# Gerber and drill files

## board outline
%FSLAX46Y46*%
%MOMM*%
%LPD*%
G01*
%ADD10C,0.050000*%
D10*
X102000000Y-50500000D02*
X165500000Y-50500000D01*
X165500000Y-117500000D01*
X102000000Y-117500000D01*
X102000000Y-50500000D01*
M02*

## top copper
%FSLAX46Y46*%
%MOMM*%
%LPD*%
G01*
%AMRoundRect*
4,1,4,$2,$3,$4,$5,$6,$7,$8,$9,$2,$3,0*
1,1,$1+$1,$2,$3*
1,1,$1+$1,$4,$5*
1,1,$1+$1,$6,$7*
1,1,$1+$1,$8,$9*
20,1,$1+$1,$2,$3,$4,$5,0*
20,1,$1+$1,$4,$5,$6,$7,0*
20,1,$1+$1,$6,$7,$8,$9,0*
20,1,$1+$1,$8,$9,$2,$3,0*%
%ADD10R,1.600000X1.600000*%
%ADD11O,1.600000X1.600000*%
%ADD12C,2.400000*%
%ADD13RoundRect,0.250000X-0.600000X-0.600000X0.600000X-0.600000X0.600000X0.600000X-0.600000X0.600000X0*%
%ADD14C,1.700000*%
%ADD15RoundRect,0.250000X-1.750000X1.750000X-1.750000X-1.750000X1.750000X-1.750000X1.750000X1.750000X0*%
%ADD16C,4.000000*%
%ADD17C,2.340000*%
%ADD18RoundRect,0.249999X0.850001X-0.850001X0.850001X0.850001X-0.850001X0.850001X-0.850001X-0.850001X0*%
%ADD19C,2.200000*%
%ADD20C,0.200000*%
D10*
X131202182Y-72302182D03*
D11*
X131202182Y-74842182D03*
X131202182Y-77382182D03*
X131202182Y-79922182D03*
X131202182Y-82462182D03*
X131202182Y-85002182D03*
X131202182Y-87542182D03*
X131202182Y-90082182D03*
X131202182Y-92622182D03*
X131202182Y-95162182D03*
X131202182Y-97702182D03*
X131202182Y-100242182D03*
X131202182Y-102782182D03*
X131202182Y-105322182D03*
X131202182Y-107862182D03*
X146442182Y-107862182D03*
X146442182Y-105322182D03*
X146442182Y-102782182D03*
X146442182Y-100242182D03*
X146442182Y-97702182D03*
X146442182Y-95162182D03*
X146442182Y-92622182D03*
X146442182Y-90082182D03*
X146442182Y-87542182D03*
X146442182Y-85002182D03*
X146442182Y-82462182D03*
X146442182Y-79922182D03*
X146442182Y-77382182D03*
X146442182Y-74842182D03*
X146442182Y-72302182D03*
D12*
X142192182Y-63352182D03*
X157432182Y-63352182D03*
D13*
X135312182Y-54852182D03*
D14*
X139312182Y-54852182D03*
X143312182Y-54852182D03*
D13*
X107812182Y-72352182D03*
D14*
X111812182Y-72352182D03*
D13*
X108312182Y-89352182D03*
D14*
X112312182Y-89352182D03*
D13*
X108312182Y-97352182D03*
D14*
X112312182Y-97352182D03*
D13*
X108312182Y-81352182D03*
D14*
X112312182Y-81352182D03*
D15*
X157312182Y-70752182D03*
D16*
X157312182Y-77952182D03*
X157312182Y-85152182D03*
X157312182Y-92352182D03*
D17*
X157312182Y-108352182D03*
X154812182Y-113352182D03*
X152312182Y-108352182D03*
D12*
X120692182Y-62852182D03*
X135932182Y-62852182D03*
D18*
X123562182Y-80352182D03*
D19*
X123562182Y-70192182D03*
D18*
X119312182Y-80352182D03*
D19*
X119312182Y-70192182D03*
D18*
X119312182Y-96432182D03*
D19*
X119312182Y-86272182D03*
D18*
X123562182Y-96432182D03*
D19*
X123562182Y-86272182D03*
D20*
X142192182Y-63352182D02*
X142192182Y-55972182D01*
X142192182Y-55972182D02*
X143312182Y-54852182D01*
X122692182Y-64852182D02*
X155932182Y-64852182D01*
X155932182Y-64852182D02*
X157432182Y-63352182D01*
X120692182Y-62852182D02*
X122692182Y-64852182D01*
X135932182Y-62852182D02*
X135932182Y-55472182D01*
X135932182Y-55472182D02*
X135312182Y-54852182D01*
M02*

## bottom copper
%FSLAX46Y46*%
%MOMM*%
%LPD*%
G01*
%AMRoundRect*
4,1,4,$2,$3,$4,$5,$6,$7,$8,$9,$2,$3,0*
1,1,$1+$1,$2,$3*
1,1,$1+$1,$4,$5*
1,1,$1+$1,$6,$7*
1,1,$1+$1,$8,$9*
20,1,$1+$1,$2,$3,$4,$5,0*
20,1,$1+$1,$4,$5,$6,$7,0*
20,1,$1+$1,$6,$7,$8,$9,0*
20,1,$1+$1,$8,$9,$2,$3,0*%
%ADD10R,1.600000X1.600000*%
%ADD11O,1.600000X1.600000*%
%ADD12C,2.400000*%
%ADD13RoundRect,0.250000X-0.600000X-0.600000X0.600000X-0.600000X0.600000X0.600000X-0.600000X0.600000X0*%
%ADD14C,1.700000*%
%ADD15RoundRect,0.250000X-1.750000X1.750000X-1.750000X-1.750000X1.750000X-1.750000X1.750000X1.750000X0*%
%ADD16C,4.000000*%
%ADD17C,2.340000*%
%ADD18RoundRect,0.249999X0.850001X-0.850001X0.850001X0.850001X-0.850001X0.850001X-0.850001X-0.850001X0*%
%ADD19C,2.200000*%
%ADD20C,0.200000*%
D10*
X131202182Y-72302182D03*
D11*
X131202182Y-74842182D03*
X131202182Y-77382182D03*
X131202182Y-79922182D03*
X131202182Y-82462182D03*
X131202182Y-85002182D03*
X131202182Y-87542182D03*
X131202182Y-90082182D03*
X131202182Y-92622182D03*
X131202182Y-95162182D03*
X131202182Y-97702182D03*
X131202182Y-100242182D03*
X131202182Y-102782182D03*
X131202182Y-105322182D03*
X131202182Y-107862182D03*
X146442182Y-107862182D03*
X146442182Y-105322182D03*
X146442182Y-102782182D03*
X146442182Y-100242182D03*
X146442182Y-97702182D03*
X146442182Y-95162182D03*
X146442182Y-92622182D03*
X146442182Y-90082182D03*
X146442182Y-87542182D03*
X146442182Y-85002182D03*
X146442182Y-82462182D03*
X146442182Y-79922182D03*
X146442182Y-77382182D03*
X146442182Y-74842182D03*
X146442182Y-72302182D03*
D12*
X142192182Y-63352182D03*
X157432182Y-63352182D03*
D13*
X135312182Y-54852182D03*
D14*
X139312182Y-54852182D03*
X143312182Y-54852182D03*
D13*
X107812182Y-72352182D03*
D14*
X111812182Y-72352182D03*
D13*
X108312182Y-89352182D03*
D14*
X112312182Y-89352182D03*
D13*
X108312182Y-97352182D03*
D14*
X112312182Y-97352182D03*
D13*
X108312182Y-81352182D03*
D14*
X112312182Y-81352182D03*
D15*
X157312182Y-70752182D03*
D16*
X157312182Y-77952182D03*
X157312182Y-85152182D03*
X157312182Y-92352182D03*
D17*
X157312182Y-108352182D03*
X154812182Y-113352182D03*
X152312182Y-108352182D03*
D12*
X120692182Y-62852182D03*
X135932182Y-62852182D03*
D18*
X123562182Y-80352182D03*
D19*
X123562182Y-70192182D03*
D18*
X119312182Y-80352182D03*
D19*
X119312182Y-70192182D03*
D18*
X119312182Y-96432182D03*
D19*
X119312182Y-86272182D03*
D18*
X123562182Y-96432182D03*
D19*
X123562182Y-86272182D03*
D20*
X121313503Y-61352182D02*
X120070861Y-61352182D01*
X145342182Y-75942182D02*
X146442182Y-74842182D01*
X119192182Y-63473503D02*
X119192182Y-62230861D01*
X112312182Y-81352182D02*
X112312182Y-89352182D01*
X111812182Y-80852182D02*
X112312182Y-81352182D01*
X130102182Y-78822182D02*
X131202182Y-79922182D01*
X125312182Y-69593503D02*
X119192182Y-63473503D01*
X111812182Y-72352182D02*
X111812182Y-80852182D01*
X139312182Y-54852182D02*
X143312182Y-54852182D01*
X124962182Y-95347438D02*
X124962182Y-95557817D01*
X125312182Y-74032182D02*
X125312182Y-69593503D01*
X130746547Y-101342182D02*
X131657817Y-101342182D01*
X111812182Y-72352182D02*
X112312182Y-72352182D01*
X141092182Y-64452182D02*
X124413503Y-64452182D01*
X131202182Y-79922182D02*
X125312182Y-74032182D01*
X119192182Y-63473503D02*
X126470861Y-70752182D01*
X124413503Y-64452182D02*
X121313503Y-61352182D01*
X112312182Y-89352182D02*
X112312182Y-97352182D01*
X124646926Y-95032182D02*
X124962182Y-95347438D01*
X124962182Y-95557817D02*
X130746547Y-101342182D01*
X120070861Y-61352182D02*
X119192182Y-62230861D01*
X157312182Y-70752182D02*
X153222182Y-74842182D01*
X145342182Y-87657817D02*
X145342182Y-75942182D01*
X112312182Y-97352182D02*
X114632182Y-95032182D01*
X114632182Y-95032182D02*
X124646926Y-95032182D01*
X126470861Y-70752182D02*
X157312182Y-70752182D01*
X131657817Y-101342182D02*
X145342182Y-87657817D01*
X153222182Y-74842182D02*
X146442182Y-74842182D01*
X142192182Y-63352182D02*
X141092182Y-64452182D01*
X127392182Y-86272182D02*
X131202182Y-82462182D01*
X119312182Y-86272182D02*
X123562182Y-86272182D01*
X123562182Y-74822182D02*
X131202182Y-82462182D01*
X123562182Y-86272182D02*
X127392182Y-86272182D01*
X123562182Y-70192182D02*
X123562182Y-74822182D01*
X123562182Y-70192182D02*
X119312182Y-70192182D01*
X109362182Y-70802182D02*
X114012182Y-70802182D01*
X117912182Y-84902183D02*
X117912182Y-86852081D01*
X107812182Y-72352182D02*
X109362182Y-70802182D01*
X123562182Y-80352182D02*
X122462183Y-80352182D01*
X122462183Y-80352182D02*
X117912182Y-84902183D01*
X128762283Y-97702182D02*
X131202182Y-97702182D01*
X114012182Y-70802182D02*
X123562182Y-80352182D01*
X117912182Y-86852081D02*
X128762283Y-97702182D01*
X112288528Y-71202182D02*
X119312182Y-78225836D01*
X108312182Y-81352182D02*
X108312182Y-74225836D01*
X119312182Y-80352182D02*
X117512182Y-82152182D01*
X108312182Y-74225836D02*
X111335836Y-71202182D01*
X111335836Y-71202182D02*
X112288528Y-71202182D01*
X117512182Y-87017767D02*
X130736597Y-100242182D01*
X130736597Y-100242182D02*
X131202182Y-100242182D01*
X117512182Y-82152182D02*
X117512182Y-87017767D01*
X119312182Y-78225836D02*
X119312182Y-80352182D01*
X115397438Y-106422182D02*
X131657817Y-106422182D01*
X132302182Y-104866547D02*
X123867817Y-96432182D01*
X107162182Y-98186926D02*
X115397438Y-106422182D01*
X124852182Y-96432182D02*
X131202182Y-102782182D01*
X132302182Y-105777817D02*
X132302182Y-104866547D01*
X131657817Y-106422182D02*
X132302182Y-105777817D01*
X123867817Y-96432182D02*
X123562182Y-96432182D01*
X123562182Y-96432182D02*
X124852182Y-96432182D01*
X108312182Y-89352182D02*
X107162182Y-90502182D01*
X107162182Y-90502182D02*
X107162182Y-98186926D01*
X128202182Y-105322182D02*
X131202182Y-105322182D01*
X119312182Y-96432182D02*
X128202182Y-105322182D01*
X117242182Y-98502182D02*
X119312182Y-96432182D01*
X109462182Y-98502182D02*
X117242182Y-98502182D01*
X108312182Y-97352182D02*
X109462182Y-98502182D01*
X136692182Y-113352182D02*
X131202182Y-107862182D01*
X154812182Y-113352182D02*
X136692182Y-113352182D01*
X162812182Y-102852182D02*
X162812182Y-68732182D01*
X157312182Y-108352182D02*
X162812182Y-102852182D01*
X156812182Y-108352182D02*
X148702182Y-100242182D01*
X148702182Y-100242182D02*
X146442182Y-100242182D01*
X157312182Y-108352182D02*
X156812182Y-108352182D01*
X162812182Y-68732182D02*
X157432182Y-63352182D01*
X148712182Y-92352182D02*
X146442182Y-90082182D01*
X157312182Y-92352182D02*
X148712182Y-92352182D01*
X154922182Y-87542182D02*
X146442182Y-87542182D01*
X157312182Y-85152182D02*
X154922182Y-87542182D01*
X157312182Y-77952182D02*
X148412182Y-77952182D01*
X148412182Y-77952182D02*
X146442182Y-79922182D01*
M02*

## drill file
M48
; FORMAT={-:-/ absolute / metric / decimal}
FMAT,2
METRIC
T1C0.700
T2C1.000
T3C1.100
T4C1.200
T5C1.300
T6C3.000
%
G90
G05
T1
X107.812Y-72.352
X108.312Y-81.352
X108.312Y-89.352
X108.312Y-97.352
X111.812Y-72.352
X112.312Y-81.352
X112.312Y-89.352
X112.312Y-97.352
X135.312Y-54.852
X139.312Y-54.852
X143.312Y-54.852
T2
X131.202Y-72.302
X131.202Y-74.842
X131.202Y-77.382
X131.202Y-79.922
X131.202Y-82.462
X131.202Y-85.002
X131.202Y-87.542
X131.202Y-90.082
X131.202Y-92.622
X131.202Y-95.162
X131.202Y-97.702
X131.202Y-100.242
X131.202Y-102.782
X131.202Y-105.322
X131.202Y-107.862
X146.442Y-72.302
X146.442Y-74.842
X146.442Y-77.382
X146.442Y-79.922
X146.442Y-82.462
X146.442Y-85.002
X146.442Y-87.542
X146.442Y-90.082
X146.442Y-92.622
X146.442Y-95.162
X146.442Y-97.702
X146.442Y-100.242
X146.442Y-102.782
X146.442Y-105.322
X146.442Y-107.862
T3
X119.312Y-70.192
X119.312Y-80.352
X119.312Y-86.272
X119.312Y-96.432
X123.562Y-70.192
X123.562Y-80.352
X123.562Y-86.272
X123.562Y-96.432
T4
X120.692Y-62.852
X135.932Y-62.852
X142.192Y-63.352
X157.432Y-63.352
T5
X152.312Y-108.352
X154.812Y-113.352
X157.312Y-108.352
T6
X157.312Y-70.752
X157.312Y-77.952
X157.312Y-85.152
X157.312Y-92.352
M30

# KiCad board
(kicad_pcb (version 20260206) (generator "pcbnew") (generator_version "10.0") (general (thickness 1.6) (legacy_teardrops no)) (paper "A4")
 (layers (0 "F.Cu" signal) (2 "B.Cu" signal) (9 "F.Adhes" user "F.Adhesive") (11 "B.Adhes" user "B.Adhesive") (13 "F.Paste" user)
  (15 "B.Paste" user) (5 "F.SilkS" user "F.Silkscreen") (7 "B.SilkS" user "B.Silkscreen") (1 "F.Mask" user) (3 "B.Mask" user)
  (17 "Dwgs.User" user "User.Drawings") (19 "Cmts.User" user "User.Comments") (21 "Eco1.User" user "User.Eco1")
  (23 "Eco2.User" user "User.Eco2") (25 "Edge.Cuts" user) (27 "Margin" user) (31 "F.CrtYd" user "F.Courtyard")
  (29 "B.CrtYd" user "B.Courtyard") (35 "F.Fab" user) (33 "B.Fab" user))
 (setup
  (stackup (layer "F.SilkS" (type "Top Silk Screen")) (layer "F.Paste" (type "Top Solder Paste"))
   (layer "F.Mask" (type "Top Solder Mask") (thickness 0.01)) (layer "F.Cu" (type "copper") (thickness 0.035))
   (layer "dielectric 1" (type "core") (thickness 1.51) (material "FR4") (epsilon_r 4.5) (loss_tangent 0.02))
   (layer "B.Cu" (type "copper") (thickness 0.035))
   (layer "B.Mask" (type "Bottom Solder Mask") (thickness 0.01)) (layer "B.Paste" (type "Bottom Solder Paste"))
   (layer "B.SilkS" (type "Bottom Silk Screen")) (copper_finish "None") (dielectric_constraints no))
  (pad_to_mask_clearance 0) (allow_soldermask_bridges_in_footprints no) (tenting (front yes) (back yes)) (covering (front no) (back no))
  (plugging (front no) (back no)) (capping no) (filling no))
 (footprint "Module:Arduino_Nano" (layer "F.Cu") (at 131.202182 72.302182)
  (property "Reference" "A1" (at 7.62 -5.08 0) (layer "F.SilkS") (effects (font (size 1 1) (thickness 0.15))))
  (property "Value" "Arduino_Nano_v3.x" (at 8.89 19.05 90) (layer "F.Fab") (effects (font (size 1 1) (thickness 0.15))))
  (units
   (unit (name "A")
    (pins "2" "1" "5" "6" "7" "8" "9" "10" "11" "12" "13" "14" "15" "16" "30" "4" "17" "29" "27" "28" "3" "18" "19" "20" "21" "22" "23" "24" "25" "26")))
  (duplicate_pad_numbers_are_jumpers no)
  (pad "1" thru_hole rect (at 0 0) (size 1.6 1.6) (drill 1) (layers "*.Cu" "*.Mask") (remove_unused_layers no)
   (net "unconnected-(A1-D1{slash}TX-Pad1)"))
  (pad "2" thru_hole oval (at 0 2.54) (size 1.6 1.6) (drill 1) (layers "*.Cu" "*.Mask") (remove_unused_layers no)
   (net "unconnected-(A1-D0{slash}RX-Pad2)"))
  (pad "3" thru_hole oval (at 0 5.08) (size 1.6 1.6) (drill 1) (layers "*.Cu" "*.Mask") (remove_unused_layers no)
   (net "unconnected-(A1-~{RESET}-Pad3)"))
  (pad "4" thru_hole oval (at 0 7.62) (size 1.6 1.6) (drill 1) (layers "*.Cu" "*.Mask") (remove_unused_layers no) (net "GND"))
  (pad "5" thru_hole oval (at 0 10.16) (size 1.6 1.6) (drill 1) (layers "*.Cu" "*.Mask") (remove_unused_layers no) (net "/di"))
  (pad "6" thru_hole oval (at 0 12.7) (size 1.6 1.6) (drill 1) (layers "*.Cu" "*.Mask") (remove_unused_layers no)
   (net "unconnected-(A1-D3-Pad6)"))
  (pad "7" thru_hole oval (at 0 15.24) (size 1.6 1.6) (drill 1) (layers "*.Cu" "*.Mask") (remove_unused_layers no)
   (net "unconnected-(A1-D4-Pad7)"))
  (pad "8" thru_hole oval (at 0 17.78) (size 1.6 1.6) (drill 1) (layers "*.Cu" "*.Mask") (remove_unused_layers no)
   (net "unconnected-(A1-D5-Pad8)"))
  (pad "9" thru_hole oval (at 0 20.32) (size 1.6 1.6) (drill 1) (layers "*.Cu" "*.Mask") (remove_unused_layers no)
   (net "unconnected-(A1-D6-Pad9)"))
  (pad "10" thru_hole oval (at 0 22.86) (size 1.6 1.6) (drill 1) (layers "*.Cu" "*.Mask") (remove_unused_layers no)
   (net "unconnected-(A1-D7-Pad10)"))
  (pad "11" thru_hole oval (at 0 25.4) (size 1.6 1.6) (drill 1) (layers "*.Cu" "*.Mask") (remove_unused_layers no) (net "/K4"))
  (pad "12" thru_hole oval (at 0 27.94) (size 1.6 1.6) (drill 1) (layers "*.Cu" "*.Mask") (remove_unused_layers no) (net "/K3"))
  (pad "13" thru_hole oval (at 0 30.48) (size 1.6 1.6) (drill 1) (layers "*.Cu" "*.Mask") (remove_unused_layers no) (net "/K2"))
  (pad "14" thru_hole oval (at 0 33.02) (size 1.6 1.6) (drill 1) (layers "*.Cu" "*.Mask") (remove_unused_layers no) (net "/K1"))
  (pad "15" thru_hole oval (at 0 35.56) (size 1.6 1.6) (drill 1) (layers "*.Cu" "*.Mask") (remove_unused_layers no) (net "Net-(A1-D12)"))
  (pad "16" thru_hole oval (at 15.24 35.56) (size 1.6 1.6) (drill 1) (layers "*.Cu" "*.Mask") (remove_unused_layers no)
   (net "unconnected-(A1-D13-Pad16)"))
  (pad "17" thru_hole oval (at 15.24 33.02) (size 1.6 1.6) (drill 1) (layers "*.Cu" "*.Mask") (remove_unused_layers no)
   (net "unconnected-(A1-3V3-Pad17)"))
  (pad "18" thru_hole oval (at 15.24 30.48) (size 1.6 1.6) (drill 1) (layers "*.Cu" "*.Mask") (remove_unused_layers no)
   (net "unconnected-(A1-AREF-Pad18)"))
  (pad "19" thru_hole oval (at 15.24 27.94) (size 1.6 1.6) (drill 1) (layers "*.Cu" "*.Mask") (remove_unused_layers no) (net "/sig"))
  (pad "20" thru_hole oval (at 15.24 25.4) (size 1.6 1.6) (drill 1) (layers "*.Cu" "*.Mask") (remove_unused_layers no)
   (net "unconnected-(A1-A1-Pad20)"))
  (pad "21" thru_hole oval (at 15.24 22.86) (size 1.6 1.6) (drill 1) (layers "*.Cu" "*.Mask") (remove_unused_layers no)
   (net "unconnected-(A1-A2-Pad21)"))
  (pad "22" thru_hole oval (at 15.24 20.32) (size 1.6 1.6) (drill 1) (layers "*.Cu" "*.Mask") (remove_unused_layers no)
   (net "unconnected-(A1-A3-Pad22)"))
  (pad "23" thru_hole oval (at 15.24 17.78) (size 1.6 1.6) (drill 1) (layers "*.Cu" "*.Mask") (remove_unused_layers no) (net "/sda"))
  (pad "24" thru_hole oval (at 15.24 15.24) (size 1.6 1.6) (drill 1) (layers "*.Cu" "*.Mask") (remove_unused_layers no) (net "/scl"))
  (pad "25" thru_hole oval (at 15.24 12.7) (size 1.6 1.6) (drill 1) (layers "*.Cu" "*.Mask") (remove_unused_layers no)
   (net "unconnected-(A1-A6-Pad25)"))
  (pad "26" thru_hole oval (at 15.24 10.16) (size 1.6 1.6) (drill 1) (layers "*.Cu" "*.Mask") (remove_unused_layers no)
   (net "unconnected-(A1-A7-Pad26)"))
  (pad "27" thru_hole oval (at 15.24 7.62) (size 1.6 1.6) (drill 1) (layers "*.Cu" "*.Mask") (remove_unused_layers no) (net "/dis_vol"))
  (pad "28" thru_hole oval (at 15.24 5.08) (size 1.6 1.6) (drill 1) (layers "*.Cu" "*.Mask") (remove_unused_layers no)
   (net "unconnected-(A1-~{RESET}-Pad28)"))
  (pad "29" thru_hole oval (at 15.24 2.54) (size 1.6 1.6) (drill 1) (layers "*.Cu" "*.Mask") (remove_unused_layers no) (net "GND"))
  (pad "30" thru_hole oval (at 15.24 0) (size 1.6 1.6) (drill 1) (layers "*.Cu" "*.Mask") (remove_unused_layers no) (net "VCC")))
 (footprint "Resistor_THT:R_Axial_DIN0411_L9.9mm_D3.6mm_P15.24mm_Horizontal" (layer "F.Cu") (at 142.192182 63.352182)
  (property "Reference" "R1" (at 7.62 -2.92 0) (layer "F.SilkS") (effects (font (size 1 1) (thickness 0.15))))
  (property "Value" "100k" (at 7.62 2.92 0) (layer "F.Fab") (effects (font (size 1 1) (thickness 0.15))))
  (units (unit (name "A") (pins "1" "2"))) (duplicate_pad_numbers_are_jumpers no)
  (pad "1" thru_hole circle (at 0 0) (size 2.4 2.4) (drill 1.2) (layers "*.Cu" "*.Mask") (remove_unused_layers no) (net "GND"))
  (pad "2" thru_hole circle (at 15.24 0) (size 2.4 2.4) (drill 1.2) (layers "*.Cu" "*.Mask") (remove_unused_layers no) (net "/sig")))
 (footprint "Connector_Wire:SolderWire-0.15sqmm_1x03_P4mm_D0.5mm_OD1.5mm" (layer "F.Cu") (at 135.312182 54.852182)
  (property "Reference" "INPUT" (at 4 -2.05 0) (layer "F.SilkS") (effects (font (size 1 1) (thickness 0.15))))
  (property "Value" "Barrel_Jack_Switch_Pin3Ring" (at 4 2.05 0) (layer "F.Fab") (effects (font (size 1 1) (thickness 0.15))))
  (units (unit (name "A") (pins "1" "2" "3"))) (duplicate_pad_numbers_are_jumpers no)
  (pad "1" thru_hole roundrect (at 0 0) (size 1.7 1.7) (drill 0.7) (layers "*.Cu" "*.Mask") (remove_unused_layers no)
   (roundrect_rratio 0.147059) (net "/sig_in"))
  (pad "2" thru_hole circle (at 4 0) (size 1.7 1.7) (drill 0.7) (layers "*.Cu" "*.Mask") (remove_unused_layers no) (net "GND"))
  (pad "3" thru_hole circle (at 8 0) (size 1.7 1.7) (drill 0.7) (layers "*.Cu" "*.Mask") (remove_unused_layers no) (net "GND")))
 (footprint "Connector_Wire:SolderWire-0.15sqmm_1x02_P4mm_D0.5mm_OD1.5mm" (layer "F.Cu") (at 107.812182 72.352182)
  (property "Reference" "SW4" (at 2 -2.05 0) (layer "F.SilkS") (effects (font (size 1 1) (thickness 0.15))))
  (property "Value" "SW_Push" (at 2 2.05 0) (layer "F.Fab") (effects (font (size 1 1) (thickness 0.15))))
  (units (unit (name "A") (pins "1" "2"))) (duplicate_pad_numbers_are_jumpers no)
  (pad "1" thru_hole roundrect (at 0 0) (size 1.7 1.7) (drill 0.7) (layers "*.Cu" "*.Mask") (remove_unused_layers no)
   (roundrect_rratio 0.147059) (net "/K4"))
  (pad "2" thru_hole circle (at 4 0) (size 1.7 1.7) (drill 0.7) (layers "*.Cu" "*.Mask") (remove_unused_layers no) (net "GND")))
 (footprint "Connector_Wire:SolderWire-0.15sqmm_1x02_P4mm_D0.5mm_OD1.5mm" (layer "F.Cu") (at 108.312182 89.352182)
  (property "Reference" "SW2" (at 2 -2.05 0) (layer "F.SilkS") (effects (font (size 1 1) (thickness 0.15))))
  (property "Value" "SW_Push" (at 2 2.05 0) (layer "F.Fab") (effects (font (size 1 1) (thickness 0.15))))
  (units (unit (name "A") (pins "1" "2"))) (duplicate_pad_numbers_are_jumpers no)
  (pad "1" thru_hole roundrect (at 0 0) (size 1.7 1.7) (drill 0.7) (layers "*.Cu" "*.Mask") (remove_unused_layers no)
   (roundrect_rratio 0.147059) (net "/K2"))
  (pad "2" thru_hole circle (at 4 0) (size 1.7 1.7) (drill 0.7) (layers "*.Cu" "*.Mask") (remove_unused_layers no) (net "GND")))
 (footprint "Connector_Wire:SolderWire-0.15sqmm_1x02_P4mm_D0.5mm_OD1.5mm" (layer "F.Cu") (at 108.312182 97.352182)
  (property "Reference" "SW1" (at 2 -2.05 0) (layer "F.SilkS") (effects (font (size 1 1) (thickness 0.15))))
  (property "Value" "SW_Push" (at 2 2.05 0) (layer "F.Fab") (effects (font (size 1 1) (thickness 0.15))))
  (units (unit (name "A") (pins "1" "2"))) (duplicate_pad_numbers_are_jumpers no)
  (pad "1" thru_hole roundrect (at 0 0) (size 1.7 1.7) (drill 0.7) (layers "*.Cu" "*.Mask") (remove_unused_layers no)
   (roundrect_rratio 0.147059) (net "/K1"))
  (pad "2" thru_hole circle (at 4 0) (size 1.7 1.7) (drill 0.7) (layers "*.Cu" "*.Mask") (remove_unused_layers no) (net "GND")))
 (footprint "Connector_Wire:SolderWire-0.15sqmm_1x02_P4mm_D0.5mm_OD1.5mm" (layer "F.Cu") (at 108.312182 81.352182)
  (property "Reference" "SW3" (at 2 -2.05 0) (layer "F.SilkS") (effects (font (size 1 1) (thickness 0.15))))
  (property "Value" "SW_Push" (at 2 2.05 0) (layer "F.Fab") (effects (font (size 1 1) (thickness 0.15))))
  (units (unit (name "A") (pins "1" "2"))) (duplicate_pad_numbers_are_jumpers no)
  (pad "1" thru_hole roundrect (at 0 0) (size 1.7 1.7) (drill 0.7) (layers "*.Cu" "*.Mask") (remove_unused_layers no)
   (roundrect_rratio 0.147059) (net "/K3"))
  (pad "2" thru_hole circle (at 4 0) (size 1.7 1.7) (drill 0.7) (layers "*.Cu" "*.Mask") (remove_unused_layers no) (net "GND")))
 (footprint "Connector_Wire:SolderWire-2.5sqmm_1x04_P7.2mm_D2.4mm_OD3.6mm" (layer "F.Cu") (at 157.312182 70.752182 -90)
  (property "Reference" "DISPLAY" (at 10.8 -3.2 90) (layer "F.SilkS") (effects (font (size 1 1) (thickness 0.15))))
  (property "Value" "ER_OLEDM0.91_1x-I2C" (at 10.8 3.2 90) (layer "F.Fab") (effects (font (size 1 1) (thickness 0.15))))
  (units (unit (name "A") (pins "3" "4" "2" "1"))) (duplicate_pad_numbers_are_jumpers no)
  (pad "1" thru_hole roundrect (at 0 0 270) (size 4 4) (drill 3) (layers "*.Cu" "*.Mask") (remove_unused_layers no)
   (roundrect_rratio 0.0625) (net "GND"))
  (pad "2" thru_hole circle (at 7.2 0 270) (size 4 4) (drill 3) (layers "*.Cu" "*.Mask") (remove_unused_layers no) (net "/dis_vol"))
  (pad "3" thru_hole circle (at 14.4 0 270) (size 4 4) (drill 3) (layers "*.Cu" "*.Mask") (remove_unused_layers no) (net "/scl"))
  (pad "4" thru_hole circle (at 21.6 0 270) (size 4 4) (drill 3) (layers "*.Cu" "*.Mask") (remove_unused_layers no) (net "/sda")))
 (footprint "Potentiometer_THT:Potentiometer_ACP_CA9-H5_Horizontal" (layer "F.Cu") (at 157.312182 108.352182 -90)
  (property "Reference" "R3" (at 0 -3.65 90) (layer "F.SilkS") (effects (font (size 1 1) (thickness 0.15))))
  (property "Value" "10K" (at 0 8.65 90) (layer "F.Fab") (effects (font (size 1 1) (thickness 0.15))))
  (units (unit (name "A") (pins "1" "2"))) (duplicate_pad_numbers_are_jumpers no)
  (pad "1" thru_hole circle (at 0 0 270) (size 2.34 2.34) (drill 1.3) (layers "*.Cu" "*.Mask") (remove_unused_layers no) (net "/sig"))
  (pad "2" thru_hole circle (at 5 2.5 270) (size 2.34 2.34) (drill 1.3) (layers "*.Cu" "*.Mask") (remove_unused_layers no)
   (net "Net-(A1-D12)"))
  (pad "3" thru_hole circle (at 0 5 270) (size 2.34 2.34) (drill 1.3) (layers "*.Cu" "*.Mask") (remove_unused_layers no)))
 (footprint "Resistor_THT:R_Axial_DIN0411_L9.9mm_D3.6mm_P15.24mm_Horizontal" (layer "F.Cu") (at 120.692182 62.852182)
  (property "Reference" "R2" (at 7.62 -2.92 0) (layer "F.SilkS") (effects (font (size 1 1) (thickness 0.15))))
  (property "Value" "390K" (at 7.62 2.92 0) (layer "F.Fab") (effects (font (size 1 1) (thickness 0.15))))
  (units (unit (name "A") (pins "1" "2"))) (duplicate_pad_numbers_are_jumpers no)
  (pad "1" thru_hole circle (at 0 0) (size 2.4 2.4) (drill 1.2) (layers "*.Cu" "*.Mask") (remove_unused_layers no) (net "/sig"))
  (pad "2" thru_hole circle (at 15.24 0) (size 2.4 2.4) (drill 1.2) (layers "*.Cu" "*.Mask") (remove_unused_layers no) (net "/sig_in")))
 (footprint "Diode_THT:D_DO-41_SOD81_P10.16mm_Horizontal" (layer "F.Cu") (at 123.562182 80.352182 90)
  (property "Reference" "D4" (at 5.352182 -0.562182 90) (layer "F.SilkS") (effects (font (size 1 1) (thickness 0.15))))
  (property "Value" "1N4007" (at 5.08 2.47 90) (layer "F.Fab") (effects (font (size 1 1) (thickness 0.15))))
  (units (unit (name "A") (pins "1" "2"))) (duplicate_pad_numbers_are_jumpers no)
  (pad "1" thru_hole roundrect (at 0 0 90) (size 2.2 2.2) (drill 1.1) (layers "*.Cu" "*.Mask") (remove_unused_layers no)
   (roundrect_rratio 0.113636) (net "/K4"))
  (pad "2" thru_hole circle (at 10.16 0 90) (size 2.2 2.2) (drill 1.1) (layers "*.Cu" "*.Mask") (remove_unused_layers no) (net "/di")))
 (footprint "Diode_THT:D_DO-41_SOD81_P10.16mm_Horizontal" (layer "F.Cu") (at 119.312182 80.352182 90)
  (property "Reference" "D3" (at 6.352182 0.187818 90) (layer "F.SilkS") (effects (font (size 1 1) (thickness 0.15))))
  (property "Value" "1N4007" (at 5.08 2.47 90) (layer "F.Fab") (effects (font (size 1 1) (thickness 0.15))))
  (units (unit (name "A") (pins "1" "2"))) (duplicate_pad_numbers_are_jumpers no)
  (pad "1" thru_hole roundrect (at 0 0 90) (size 2.2 2.2) (drill 1.1) (layers "*.Cu" "*.Mask") (remove_unused_layers no)
   (roundrect_rratio 0.113636) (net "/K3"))
  (pad "2" thru_hole circle (at 10.16 0 90) (size 2.2 2.2) (drill 1.1) (layers "*.Cu" "*.Mask") (remove_unused_layers no) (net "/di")))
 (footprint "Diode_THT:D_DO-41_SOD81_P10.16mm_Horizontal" (layer "F.Cu") (at 119.312182 96.432182 90)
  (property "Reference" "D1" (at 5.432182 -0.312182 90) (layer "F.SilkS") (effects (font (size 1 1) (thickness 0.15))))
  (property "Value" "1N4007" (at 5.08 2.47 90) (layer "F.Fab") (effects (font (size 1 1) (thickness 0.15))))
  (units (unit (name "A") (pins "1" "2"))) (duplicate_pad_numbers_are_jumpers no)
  (pad "1" thru_hole roundrect (at 0 0 90) (size 2.2 2.2) (drill 1.1) (layers "*.Cu" "*.Mask") (remove_unused_layers no)
   (roundrect_rratio 0.113636) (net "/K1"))
  (pad "2" thru_hole circle (at 10.16 0 90) (size 2.2 2.2) (drill 1.1) (layers "*.Cu" "*.Mask") (remove_unused_layers no) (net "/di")))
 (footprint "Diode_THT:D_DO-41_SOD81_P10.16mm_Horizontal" (layer "F.Cu") (at 123.562182 96.432182 90)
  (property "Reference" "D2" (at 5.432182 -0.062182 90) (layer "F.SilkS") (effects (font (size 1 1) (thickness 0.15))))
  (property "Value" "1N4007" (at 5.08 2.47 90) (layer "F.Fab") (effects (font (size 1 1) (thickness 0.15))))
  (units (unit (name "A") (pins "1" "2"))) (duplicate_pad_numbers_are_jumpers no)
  (pad "1" thru_hole roundrect (at 0 0 90) (size 2.2 2.2) (drill 1.1) (layers "*.Cu" "*.Mask") (remove_unused_layers no)
   (roundrect_rratio 0.113636) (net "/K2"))
  (pad "2" thru_hole circle (at 10.16 0 90) (size 2.2 2.2) (drill 1.1) (layers "*.Cu" "*.Mask") (remove_unused_layers no) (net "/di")))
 (gr_rect (start 102 50.5) (end 165.5 117.5) (stroke (width 0.05) (type default)) (fill no) (layer "Edge.Cuts"))
 (segment (start 142.192182 63.352182) (end 142.192182 55.972182) (width 0.2) (layer "F.Cu") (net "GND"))
 (segment (start 142.192182 55.972182) (end 143.312182 54.852182) (width 0.2) (layer "F.Cu") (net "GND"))
 (segment (start 121.313503 61.352182) (end 120.070861 61.352182) (width 0.2) (layer "B.Cu") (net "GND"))
 (segment (start 145.342182 75.942182) (end 146.442182 74.842182) (width 0.2) (layer "B.Cu") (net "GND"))
 (segment (start 119.192182 63.473503) (end 119.192182 62.230861) (width 0.2) (layer "B.Cu") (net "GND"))
 (segment (start 112.312182 81.352182) (end 112.312182 89.352182) (width 0.2) (layer "B.Cu") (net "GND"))
 (segment (start 111.812182 80.852182) (end 112.312182 81.352182) (width 0.2) (layer "B.Cu") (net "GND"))
 (segment (start 130.102182 78.822182) (end 131.202182 79.922182) (width 0.2) (layer "B.Cu") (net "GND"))
 (segment (start 125.312182 69.593503) (end 119.192182 63.473503) (width 0.2) (layer "B.Cu") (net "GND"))
 (segment (start 111.812182 72.352182) (end 111.812182 80.852182) (width 0.2) (layer "B.Cu") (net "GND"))
 (segment (start 139.312182 54.852182) (end 143.312182 54.852182) (width 0.2) (layer "B.Cu") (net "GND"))
 (segment (start 124.962182 95.347438) (end 124.962182 95.557817) (width 0.2) (layer "B.Cu") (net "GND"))
 (segment (start 125.312182 74.032182) (end 125.312182 69.593503) (width 0.2) (layer "B.Cu") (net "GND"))
 (segment (start 130.746547 101.342182) (end 131.657817 101.342182) (width 0.2) (layer "B.Cu") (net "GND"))
 (segment (start 111.812182 72.352182) (end 112.312182 72.352182) (width 0.2) (layer "B.Cu") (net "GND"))
 (segment (start 141.092182 64.452182) (end 124.413503 64.452182) (width 0.2) (layer "B.Cu") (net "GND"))
 (segment (start 131.202182 79.922182) (end 125.312182 74.032182) (width 0.2) (layer "B.Cu") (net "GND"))
 (segment (start 119.192182 63.473503) (end 126.470861 70.752182) (width 0.2) (layer "B.Cu") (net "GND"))
 (segment (start 124.413503 64.452182) (end 121.313503 61.352182) (width 0.2) (layer "B.Cu") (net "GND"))
 (segment (start 112.312182 89.352182) (end 112.312182 97.352182) (width 0.2) (layer "B.Cu") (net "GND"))
 (segment (start 124.646926 95.032182) (end 124.962182 95.347438) (width 0.2) (layer "B.Cu") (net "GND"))
 (segment (start 124.962182 95.557817) (end 130.746547 101.342182) (width 0.2) (layer "B.Cu") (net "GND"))
 (segment (start 120.070861 61.352182) (end 119.192182 62.230861) (width 0.2) (layer "B.Cu") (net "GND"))
 (segment (start 157.312182 70.752182) (end 153.222182 74.842182) (width 0.2) (layer "B.Cu") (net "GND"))
 (segment (start 145.342182 87.657817) (end 145.342182 75.942182) (width 0.2) (layer "B.Cu") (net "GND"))
 (segment (start 112.312182 97.352182) (end 114.632182 95.032182) (width 0.2) (layer "B.Cu") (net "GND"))
 (segment (start 114.632182 95.032182) (end 124.646926 95.032182) (width 0.2) (layer "B.Cu") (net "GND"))
 (segment (start 126.470861 70.752182) (end 157.312182 70.752182) (width 0.2) (layer "B.Cu") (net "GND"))
 (segment (start 131.657817 101.342182) (end 145.342182 87.657817) (width 0.2) (layer "B.Cu") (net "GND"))
 (segment (start 153.222182 74.842182) (end 146.442182 74.842182) (width 0.2) (layer "B.Cu") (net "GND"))
 (segment (start 142.192182 63.352182) (end 141.092182 64.452182) (width 0.2) (layer "B.Cu") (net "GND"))
 (segment (start 127.392182 86.272182) (end 131.202182 82.462182) (width 0.2) (layer "B.Cu") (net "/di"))
 (segment (start 119.312182 86.272182) (end 123.562182 86.272182) (width 0.2) (layer "B.Cu") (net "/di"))
 (segment (start 123.562182 74.822182) (end 131.202182 82.462182) (width 0.2) (layer "B.Cu") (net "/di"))
 (segment (start 123.562182 86.272182) (end 127.392182 86.272182) (width 0.2) (layer "B.Cu") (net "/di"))
 (segment (start 123.562182 70.192182) (end 123.562182 74.822182) (width 0.2) (layer "B.Cu") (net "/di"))
 (segment (start 123.562182 70.192182) (end 119.312182 70.192182) (width 0.2) (layer "B.Cu") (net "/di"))
 (segment (start 109.362182 70.802182) (end 114.012182 70.802182) (width 0.2) (layer "B.Cu") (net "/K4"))
 (segment (start 117.912182 84.902183) (end 117.912182 86.852081) (width 0.2) (layer "B.Cu") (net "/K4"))
 (segment (start 107.812182 72.352182) (end 109.362182 70.802182) (width 0.2) (layer "B.Cu") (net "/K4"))
 (segment (start 123.562182 80.352182) (end 122.462183 80.352182) (width 0.2) (layer "B.Cu") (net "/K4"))
 (segment (start 122.462183 80.352182) (end 117.912182 84.902183) (width 0.2) (layer "B.Cu") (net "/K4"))
 (segment (start 128.762283 97.702182) (end 131.202182 97.702182) (width 0.2) (layer "B.Cu") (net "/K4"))
 (segment (start 114.012182 70.802182) (end 123.562182 80.352182) (width 0.2) (layer "B.Cu") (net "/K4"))
 (segment (start 117.912182 86.852081) (end 128.762283 97.702182) (width 0.2) (layer "B.Cu") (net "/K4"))
 (segment (start 112.288528 71.202182) (end 119.312182 78.225836) (width 0.2) (layer "B.Cu") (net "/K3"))
 (segment (start 108.312182 81.352182) (end 108.312182 74.225836) (width 0.2) (layer "B.Cu") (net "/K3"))
 (segment (start 119.312182 80.352182) (end 117.512182 82.152182) (width 0.2) (layer "B.Cu") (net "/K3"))
 (segment (start 108.312182 74.225836) (end 111.335836 71.202182) (width 0.2) (layer "B.Cu") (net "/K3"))
 (segment (start 111.335836 71.202182) (end 112.288528 71.202182) (width 0.2) (layer "B.Cu") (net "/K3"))
 (segment (start 117.512182 87.017767) (end 130.736597 100.242182) (width 0.2) (layer "B.Cu") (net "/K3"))
 (segment (start 130.736597 100.242182) (end 131.202182 100.242182) (width 0.2) (layer "B.Cu") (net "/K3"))
 (segment (start 117.512182 82.152182) (end 117.512182 87.017767) (width 0.2) (layer "B.Cu") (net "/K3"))
 (segment (start 119.312182 78.225836) (end 119.312182 80.352182) (width 0.2) (layer "B.Cu") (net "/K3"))
 (segment (start 115.397438 106.422182) (end 131.657817 106.422182) (width 0.2) (layer "B.Cu") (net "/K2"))
 (segment (start 132.302182 104.866547) (end 123.867817 96.432182) (width 0.2) (layer "B.Cu") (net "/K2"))
 (segment (start 107.162182 98.186926) (end 115.397438 106.422182) (width 0.2) (layer "B.Cu") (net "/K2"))
 (segment (start 124.852182 96.432182) (end 131.202182 102.782182) (width 0.2) (layer "B.Cu") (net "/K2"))
 (segment (start 132.302182 105.777817) (end 132.302182 104.866547) (width 0.2) (layer "B.Cu") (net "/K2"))
 (segment (start 131.657817 106.422182) (end 132.302182 105.777817) (width 0.2) (layer "B.Cu") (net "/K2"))
 (segment (start 123.867817 96.432182) (end 123.562182 96.432182) (width 0.2) (layer "B.Cu") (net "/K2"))
 (segment (start 123.562182 96.432182) (end 124.852182 96.432182) (width 0.2) (layer "B.Cu") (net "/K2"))
 (segment (start 108.312182 89.352182) (end 107.162182 90.502182) (width 0.2) (layer "B.Cu") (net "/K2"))
 (segment (start 107.162182 90.502182) (end 107.162182 98.186926) (width 0.2) (layer "B.Cu") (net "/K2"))
 (segment (start 128.202182 105.322182) (end 131.202182 105.322182) (width 0.2) (layer "B.Cu") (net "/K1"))
 (segment (start 119.312182 96.432182) (end 128.202182 105.322182) (width 0.2) (layer "B.Cu") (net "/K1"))
 (segment (start 117.242182 98.502182) (end 119.312182 96.432182) (width 0.2) (layer "B.Cu") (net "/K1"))
 (segment (start 109.462182 98.502182) (end 117.242182 98.502182) (width 0.2) (layer "B.Cu") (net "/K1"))
 (segment (start 108.312182 97.352182) (end 109.462182 98.502182) (width 0.2) (layer "B.Cu") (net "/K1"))
 (segment (start 136.692182 113.352182) (end 131.202182 107.862182) (width 0.2) (layer "B.Cu") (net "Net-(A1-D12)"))
 (segment (start 154.812182 113.352182) (end 136.692182 113.352182) (width 0.2) (layer "B.Cu") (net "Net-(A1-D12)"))
 (segment (start 122.692182 64.852182) (end 155.932182 64.852182) (width 0.2) (layer "F.Cu") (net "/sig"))
 (segment (start 155.932182 64.852182) (end 157.432182 63.352182) (width 0.2) (layer "F.Cu") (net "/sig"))
 (segment (start 120.692182 62.852182) (end 122.692182 64.852182) (width 0.2) (layer "F.Cu") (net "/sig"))
 (segment (start 162.812182 102.852182) (end 162.812182 68.732182) (width 0.2) (layer "B.Cu") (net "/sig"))
 (segment (start 157.312182 108.352182) (end 162.812182 102.852182) (width 0.2) (layer "B.Cu") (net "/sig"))
 (segment (start 156.812182 108.352182) (end 148.702182 100.242182) (width 0.2) (layer "B.Cu") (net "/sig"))
 (segment (start 148.702182 100.242182) (end 146.442182 100.242182) (width 0.2) (layer "B.Cu") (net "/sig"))
 (segment (start 157.312182 108.352182) (end 156.812182 108.352182) (width 0.2) (layer "B.Cu") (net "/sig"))
 (segment (start 162.812182 68.732182) (end 157.432182 63.352182) (width 0.2) (layer "B.Cu") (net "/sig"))
 (segment (start 148.712182 92.352182) (end 146.442182 90.082182) (width 0.2) (layer "B.Cu") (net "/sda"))
 (segment (start 157.312182 92.352182) (end 148.712182 92.352182) (width 0.2) (layer "B.Cu") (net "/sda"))
 (segment (start 154.922182 87.542182) (end 146.442182 87.542182) (width 0.2) (layer "B.Cu") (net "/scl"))
 (segment (start 157.312182 85.152182) (end 154.922182 87.542182) (width 0.2) (layer "B.Cu") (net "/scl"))
 (segment (start 157.312182 77.952182) (end 148.412182 77.952182) (width 0.2) (layer "B.Cu") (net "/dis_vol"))
 (segment (start 148.412182 77.952182) (end 146.442182 79.922182) (width 0.2) (layer "B.Cu") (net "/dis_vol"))
 (segment (start 135.932182 62.852182) (end 135.932182 55.472182) (width 0.2) (layer "F.Cu") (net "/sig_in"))
 (segment (start 135.932182 55.472182) (end 135.312182 54.852182) (width 0.2) (layer "F.Cu") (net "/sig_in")))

